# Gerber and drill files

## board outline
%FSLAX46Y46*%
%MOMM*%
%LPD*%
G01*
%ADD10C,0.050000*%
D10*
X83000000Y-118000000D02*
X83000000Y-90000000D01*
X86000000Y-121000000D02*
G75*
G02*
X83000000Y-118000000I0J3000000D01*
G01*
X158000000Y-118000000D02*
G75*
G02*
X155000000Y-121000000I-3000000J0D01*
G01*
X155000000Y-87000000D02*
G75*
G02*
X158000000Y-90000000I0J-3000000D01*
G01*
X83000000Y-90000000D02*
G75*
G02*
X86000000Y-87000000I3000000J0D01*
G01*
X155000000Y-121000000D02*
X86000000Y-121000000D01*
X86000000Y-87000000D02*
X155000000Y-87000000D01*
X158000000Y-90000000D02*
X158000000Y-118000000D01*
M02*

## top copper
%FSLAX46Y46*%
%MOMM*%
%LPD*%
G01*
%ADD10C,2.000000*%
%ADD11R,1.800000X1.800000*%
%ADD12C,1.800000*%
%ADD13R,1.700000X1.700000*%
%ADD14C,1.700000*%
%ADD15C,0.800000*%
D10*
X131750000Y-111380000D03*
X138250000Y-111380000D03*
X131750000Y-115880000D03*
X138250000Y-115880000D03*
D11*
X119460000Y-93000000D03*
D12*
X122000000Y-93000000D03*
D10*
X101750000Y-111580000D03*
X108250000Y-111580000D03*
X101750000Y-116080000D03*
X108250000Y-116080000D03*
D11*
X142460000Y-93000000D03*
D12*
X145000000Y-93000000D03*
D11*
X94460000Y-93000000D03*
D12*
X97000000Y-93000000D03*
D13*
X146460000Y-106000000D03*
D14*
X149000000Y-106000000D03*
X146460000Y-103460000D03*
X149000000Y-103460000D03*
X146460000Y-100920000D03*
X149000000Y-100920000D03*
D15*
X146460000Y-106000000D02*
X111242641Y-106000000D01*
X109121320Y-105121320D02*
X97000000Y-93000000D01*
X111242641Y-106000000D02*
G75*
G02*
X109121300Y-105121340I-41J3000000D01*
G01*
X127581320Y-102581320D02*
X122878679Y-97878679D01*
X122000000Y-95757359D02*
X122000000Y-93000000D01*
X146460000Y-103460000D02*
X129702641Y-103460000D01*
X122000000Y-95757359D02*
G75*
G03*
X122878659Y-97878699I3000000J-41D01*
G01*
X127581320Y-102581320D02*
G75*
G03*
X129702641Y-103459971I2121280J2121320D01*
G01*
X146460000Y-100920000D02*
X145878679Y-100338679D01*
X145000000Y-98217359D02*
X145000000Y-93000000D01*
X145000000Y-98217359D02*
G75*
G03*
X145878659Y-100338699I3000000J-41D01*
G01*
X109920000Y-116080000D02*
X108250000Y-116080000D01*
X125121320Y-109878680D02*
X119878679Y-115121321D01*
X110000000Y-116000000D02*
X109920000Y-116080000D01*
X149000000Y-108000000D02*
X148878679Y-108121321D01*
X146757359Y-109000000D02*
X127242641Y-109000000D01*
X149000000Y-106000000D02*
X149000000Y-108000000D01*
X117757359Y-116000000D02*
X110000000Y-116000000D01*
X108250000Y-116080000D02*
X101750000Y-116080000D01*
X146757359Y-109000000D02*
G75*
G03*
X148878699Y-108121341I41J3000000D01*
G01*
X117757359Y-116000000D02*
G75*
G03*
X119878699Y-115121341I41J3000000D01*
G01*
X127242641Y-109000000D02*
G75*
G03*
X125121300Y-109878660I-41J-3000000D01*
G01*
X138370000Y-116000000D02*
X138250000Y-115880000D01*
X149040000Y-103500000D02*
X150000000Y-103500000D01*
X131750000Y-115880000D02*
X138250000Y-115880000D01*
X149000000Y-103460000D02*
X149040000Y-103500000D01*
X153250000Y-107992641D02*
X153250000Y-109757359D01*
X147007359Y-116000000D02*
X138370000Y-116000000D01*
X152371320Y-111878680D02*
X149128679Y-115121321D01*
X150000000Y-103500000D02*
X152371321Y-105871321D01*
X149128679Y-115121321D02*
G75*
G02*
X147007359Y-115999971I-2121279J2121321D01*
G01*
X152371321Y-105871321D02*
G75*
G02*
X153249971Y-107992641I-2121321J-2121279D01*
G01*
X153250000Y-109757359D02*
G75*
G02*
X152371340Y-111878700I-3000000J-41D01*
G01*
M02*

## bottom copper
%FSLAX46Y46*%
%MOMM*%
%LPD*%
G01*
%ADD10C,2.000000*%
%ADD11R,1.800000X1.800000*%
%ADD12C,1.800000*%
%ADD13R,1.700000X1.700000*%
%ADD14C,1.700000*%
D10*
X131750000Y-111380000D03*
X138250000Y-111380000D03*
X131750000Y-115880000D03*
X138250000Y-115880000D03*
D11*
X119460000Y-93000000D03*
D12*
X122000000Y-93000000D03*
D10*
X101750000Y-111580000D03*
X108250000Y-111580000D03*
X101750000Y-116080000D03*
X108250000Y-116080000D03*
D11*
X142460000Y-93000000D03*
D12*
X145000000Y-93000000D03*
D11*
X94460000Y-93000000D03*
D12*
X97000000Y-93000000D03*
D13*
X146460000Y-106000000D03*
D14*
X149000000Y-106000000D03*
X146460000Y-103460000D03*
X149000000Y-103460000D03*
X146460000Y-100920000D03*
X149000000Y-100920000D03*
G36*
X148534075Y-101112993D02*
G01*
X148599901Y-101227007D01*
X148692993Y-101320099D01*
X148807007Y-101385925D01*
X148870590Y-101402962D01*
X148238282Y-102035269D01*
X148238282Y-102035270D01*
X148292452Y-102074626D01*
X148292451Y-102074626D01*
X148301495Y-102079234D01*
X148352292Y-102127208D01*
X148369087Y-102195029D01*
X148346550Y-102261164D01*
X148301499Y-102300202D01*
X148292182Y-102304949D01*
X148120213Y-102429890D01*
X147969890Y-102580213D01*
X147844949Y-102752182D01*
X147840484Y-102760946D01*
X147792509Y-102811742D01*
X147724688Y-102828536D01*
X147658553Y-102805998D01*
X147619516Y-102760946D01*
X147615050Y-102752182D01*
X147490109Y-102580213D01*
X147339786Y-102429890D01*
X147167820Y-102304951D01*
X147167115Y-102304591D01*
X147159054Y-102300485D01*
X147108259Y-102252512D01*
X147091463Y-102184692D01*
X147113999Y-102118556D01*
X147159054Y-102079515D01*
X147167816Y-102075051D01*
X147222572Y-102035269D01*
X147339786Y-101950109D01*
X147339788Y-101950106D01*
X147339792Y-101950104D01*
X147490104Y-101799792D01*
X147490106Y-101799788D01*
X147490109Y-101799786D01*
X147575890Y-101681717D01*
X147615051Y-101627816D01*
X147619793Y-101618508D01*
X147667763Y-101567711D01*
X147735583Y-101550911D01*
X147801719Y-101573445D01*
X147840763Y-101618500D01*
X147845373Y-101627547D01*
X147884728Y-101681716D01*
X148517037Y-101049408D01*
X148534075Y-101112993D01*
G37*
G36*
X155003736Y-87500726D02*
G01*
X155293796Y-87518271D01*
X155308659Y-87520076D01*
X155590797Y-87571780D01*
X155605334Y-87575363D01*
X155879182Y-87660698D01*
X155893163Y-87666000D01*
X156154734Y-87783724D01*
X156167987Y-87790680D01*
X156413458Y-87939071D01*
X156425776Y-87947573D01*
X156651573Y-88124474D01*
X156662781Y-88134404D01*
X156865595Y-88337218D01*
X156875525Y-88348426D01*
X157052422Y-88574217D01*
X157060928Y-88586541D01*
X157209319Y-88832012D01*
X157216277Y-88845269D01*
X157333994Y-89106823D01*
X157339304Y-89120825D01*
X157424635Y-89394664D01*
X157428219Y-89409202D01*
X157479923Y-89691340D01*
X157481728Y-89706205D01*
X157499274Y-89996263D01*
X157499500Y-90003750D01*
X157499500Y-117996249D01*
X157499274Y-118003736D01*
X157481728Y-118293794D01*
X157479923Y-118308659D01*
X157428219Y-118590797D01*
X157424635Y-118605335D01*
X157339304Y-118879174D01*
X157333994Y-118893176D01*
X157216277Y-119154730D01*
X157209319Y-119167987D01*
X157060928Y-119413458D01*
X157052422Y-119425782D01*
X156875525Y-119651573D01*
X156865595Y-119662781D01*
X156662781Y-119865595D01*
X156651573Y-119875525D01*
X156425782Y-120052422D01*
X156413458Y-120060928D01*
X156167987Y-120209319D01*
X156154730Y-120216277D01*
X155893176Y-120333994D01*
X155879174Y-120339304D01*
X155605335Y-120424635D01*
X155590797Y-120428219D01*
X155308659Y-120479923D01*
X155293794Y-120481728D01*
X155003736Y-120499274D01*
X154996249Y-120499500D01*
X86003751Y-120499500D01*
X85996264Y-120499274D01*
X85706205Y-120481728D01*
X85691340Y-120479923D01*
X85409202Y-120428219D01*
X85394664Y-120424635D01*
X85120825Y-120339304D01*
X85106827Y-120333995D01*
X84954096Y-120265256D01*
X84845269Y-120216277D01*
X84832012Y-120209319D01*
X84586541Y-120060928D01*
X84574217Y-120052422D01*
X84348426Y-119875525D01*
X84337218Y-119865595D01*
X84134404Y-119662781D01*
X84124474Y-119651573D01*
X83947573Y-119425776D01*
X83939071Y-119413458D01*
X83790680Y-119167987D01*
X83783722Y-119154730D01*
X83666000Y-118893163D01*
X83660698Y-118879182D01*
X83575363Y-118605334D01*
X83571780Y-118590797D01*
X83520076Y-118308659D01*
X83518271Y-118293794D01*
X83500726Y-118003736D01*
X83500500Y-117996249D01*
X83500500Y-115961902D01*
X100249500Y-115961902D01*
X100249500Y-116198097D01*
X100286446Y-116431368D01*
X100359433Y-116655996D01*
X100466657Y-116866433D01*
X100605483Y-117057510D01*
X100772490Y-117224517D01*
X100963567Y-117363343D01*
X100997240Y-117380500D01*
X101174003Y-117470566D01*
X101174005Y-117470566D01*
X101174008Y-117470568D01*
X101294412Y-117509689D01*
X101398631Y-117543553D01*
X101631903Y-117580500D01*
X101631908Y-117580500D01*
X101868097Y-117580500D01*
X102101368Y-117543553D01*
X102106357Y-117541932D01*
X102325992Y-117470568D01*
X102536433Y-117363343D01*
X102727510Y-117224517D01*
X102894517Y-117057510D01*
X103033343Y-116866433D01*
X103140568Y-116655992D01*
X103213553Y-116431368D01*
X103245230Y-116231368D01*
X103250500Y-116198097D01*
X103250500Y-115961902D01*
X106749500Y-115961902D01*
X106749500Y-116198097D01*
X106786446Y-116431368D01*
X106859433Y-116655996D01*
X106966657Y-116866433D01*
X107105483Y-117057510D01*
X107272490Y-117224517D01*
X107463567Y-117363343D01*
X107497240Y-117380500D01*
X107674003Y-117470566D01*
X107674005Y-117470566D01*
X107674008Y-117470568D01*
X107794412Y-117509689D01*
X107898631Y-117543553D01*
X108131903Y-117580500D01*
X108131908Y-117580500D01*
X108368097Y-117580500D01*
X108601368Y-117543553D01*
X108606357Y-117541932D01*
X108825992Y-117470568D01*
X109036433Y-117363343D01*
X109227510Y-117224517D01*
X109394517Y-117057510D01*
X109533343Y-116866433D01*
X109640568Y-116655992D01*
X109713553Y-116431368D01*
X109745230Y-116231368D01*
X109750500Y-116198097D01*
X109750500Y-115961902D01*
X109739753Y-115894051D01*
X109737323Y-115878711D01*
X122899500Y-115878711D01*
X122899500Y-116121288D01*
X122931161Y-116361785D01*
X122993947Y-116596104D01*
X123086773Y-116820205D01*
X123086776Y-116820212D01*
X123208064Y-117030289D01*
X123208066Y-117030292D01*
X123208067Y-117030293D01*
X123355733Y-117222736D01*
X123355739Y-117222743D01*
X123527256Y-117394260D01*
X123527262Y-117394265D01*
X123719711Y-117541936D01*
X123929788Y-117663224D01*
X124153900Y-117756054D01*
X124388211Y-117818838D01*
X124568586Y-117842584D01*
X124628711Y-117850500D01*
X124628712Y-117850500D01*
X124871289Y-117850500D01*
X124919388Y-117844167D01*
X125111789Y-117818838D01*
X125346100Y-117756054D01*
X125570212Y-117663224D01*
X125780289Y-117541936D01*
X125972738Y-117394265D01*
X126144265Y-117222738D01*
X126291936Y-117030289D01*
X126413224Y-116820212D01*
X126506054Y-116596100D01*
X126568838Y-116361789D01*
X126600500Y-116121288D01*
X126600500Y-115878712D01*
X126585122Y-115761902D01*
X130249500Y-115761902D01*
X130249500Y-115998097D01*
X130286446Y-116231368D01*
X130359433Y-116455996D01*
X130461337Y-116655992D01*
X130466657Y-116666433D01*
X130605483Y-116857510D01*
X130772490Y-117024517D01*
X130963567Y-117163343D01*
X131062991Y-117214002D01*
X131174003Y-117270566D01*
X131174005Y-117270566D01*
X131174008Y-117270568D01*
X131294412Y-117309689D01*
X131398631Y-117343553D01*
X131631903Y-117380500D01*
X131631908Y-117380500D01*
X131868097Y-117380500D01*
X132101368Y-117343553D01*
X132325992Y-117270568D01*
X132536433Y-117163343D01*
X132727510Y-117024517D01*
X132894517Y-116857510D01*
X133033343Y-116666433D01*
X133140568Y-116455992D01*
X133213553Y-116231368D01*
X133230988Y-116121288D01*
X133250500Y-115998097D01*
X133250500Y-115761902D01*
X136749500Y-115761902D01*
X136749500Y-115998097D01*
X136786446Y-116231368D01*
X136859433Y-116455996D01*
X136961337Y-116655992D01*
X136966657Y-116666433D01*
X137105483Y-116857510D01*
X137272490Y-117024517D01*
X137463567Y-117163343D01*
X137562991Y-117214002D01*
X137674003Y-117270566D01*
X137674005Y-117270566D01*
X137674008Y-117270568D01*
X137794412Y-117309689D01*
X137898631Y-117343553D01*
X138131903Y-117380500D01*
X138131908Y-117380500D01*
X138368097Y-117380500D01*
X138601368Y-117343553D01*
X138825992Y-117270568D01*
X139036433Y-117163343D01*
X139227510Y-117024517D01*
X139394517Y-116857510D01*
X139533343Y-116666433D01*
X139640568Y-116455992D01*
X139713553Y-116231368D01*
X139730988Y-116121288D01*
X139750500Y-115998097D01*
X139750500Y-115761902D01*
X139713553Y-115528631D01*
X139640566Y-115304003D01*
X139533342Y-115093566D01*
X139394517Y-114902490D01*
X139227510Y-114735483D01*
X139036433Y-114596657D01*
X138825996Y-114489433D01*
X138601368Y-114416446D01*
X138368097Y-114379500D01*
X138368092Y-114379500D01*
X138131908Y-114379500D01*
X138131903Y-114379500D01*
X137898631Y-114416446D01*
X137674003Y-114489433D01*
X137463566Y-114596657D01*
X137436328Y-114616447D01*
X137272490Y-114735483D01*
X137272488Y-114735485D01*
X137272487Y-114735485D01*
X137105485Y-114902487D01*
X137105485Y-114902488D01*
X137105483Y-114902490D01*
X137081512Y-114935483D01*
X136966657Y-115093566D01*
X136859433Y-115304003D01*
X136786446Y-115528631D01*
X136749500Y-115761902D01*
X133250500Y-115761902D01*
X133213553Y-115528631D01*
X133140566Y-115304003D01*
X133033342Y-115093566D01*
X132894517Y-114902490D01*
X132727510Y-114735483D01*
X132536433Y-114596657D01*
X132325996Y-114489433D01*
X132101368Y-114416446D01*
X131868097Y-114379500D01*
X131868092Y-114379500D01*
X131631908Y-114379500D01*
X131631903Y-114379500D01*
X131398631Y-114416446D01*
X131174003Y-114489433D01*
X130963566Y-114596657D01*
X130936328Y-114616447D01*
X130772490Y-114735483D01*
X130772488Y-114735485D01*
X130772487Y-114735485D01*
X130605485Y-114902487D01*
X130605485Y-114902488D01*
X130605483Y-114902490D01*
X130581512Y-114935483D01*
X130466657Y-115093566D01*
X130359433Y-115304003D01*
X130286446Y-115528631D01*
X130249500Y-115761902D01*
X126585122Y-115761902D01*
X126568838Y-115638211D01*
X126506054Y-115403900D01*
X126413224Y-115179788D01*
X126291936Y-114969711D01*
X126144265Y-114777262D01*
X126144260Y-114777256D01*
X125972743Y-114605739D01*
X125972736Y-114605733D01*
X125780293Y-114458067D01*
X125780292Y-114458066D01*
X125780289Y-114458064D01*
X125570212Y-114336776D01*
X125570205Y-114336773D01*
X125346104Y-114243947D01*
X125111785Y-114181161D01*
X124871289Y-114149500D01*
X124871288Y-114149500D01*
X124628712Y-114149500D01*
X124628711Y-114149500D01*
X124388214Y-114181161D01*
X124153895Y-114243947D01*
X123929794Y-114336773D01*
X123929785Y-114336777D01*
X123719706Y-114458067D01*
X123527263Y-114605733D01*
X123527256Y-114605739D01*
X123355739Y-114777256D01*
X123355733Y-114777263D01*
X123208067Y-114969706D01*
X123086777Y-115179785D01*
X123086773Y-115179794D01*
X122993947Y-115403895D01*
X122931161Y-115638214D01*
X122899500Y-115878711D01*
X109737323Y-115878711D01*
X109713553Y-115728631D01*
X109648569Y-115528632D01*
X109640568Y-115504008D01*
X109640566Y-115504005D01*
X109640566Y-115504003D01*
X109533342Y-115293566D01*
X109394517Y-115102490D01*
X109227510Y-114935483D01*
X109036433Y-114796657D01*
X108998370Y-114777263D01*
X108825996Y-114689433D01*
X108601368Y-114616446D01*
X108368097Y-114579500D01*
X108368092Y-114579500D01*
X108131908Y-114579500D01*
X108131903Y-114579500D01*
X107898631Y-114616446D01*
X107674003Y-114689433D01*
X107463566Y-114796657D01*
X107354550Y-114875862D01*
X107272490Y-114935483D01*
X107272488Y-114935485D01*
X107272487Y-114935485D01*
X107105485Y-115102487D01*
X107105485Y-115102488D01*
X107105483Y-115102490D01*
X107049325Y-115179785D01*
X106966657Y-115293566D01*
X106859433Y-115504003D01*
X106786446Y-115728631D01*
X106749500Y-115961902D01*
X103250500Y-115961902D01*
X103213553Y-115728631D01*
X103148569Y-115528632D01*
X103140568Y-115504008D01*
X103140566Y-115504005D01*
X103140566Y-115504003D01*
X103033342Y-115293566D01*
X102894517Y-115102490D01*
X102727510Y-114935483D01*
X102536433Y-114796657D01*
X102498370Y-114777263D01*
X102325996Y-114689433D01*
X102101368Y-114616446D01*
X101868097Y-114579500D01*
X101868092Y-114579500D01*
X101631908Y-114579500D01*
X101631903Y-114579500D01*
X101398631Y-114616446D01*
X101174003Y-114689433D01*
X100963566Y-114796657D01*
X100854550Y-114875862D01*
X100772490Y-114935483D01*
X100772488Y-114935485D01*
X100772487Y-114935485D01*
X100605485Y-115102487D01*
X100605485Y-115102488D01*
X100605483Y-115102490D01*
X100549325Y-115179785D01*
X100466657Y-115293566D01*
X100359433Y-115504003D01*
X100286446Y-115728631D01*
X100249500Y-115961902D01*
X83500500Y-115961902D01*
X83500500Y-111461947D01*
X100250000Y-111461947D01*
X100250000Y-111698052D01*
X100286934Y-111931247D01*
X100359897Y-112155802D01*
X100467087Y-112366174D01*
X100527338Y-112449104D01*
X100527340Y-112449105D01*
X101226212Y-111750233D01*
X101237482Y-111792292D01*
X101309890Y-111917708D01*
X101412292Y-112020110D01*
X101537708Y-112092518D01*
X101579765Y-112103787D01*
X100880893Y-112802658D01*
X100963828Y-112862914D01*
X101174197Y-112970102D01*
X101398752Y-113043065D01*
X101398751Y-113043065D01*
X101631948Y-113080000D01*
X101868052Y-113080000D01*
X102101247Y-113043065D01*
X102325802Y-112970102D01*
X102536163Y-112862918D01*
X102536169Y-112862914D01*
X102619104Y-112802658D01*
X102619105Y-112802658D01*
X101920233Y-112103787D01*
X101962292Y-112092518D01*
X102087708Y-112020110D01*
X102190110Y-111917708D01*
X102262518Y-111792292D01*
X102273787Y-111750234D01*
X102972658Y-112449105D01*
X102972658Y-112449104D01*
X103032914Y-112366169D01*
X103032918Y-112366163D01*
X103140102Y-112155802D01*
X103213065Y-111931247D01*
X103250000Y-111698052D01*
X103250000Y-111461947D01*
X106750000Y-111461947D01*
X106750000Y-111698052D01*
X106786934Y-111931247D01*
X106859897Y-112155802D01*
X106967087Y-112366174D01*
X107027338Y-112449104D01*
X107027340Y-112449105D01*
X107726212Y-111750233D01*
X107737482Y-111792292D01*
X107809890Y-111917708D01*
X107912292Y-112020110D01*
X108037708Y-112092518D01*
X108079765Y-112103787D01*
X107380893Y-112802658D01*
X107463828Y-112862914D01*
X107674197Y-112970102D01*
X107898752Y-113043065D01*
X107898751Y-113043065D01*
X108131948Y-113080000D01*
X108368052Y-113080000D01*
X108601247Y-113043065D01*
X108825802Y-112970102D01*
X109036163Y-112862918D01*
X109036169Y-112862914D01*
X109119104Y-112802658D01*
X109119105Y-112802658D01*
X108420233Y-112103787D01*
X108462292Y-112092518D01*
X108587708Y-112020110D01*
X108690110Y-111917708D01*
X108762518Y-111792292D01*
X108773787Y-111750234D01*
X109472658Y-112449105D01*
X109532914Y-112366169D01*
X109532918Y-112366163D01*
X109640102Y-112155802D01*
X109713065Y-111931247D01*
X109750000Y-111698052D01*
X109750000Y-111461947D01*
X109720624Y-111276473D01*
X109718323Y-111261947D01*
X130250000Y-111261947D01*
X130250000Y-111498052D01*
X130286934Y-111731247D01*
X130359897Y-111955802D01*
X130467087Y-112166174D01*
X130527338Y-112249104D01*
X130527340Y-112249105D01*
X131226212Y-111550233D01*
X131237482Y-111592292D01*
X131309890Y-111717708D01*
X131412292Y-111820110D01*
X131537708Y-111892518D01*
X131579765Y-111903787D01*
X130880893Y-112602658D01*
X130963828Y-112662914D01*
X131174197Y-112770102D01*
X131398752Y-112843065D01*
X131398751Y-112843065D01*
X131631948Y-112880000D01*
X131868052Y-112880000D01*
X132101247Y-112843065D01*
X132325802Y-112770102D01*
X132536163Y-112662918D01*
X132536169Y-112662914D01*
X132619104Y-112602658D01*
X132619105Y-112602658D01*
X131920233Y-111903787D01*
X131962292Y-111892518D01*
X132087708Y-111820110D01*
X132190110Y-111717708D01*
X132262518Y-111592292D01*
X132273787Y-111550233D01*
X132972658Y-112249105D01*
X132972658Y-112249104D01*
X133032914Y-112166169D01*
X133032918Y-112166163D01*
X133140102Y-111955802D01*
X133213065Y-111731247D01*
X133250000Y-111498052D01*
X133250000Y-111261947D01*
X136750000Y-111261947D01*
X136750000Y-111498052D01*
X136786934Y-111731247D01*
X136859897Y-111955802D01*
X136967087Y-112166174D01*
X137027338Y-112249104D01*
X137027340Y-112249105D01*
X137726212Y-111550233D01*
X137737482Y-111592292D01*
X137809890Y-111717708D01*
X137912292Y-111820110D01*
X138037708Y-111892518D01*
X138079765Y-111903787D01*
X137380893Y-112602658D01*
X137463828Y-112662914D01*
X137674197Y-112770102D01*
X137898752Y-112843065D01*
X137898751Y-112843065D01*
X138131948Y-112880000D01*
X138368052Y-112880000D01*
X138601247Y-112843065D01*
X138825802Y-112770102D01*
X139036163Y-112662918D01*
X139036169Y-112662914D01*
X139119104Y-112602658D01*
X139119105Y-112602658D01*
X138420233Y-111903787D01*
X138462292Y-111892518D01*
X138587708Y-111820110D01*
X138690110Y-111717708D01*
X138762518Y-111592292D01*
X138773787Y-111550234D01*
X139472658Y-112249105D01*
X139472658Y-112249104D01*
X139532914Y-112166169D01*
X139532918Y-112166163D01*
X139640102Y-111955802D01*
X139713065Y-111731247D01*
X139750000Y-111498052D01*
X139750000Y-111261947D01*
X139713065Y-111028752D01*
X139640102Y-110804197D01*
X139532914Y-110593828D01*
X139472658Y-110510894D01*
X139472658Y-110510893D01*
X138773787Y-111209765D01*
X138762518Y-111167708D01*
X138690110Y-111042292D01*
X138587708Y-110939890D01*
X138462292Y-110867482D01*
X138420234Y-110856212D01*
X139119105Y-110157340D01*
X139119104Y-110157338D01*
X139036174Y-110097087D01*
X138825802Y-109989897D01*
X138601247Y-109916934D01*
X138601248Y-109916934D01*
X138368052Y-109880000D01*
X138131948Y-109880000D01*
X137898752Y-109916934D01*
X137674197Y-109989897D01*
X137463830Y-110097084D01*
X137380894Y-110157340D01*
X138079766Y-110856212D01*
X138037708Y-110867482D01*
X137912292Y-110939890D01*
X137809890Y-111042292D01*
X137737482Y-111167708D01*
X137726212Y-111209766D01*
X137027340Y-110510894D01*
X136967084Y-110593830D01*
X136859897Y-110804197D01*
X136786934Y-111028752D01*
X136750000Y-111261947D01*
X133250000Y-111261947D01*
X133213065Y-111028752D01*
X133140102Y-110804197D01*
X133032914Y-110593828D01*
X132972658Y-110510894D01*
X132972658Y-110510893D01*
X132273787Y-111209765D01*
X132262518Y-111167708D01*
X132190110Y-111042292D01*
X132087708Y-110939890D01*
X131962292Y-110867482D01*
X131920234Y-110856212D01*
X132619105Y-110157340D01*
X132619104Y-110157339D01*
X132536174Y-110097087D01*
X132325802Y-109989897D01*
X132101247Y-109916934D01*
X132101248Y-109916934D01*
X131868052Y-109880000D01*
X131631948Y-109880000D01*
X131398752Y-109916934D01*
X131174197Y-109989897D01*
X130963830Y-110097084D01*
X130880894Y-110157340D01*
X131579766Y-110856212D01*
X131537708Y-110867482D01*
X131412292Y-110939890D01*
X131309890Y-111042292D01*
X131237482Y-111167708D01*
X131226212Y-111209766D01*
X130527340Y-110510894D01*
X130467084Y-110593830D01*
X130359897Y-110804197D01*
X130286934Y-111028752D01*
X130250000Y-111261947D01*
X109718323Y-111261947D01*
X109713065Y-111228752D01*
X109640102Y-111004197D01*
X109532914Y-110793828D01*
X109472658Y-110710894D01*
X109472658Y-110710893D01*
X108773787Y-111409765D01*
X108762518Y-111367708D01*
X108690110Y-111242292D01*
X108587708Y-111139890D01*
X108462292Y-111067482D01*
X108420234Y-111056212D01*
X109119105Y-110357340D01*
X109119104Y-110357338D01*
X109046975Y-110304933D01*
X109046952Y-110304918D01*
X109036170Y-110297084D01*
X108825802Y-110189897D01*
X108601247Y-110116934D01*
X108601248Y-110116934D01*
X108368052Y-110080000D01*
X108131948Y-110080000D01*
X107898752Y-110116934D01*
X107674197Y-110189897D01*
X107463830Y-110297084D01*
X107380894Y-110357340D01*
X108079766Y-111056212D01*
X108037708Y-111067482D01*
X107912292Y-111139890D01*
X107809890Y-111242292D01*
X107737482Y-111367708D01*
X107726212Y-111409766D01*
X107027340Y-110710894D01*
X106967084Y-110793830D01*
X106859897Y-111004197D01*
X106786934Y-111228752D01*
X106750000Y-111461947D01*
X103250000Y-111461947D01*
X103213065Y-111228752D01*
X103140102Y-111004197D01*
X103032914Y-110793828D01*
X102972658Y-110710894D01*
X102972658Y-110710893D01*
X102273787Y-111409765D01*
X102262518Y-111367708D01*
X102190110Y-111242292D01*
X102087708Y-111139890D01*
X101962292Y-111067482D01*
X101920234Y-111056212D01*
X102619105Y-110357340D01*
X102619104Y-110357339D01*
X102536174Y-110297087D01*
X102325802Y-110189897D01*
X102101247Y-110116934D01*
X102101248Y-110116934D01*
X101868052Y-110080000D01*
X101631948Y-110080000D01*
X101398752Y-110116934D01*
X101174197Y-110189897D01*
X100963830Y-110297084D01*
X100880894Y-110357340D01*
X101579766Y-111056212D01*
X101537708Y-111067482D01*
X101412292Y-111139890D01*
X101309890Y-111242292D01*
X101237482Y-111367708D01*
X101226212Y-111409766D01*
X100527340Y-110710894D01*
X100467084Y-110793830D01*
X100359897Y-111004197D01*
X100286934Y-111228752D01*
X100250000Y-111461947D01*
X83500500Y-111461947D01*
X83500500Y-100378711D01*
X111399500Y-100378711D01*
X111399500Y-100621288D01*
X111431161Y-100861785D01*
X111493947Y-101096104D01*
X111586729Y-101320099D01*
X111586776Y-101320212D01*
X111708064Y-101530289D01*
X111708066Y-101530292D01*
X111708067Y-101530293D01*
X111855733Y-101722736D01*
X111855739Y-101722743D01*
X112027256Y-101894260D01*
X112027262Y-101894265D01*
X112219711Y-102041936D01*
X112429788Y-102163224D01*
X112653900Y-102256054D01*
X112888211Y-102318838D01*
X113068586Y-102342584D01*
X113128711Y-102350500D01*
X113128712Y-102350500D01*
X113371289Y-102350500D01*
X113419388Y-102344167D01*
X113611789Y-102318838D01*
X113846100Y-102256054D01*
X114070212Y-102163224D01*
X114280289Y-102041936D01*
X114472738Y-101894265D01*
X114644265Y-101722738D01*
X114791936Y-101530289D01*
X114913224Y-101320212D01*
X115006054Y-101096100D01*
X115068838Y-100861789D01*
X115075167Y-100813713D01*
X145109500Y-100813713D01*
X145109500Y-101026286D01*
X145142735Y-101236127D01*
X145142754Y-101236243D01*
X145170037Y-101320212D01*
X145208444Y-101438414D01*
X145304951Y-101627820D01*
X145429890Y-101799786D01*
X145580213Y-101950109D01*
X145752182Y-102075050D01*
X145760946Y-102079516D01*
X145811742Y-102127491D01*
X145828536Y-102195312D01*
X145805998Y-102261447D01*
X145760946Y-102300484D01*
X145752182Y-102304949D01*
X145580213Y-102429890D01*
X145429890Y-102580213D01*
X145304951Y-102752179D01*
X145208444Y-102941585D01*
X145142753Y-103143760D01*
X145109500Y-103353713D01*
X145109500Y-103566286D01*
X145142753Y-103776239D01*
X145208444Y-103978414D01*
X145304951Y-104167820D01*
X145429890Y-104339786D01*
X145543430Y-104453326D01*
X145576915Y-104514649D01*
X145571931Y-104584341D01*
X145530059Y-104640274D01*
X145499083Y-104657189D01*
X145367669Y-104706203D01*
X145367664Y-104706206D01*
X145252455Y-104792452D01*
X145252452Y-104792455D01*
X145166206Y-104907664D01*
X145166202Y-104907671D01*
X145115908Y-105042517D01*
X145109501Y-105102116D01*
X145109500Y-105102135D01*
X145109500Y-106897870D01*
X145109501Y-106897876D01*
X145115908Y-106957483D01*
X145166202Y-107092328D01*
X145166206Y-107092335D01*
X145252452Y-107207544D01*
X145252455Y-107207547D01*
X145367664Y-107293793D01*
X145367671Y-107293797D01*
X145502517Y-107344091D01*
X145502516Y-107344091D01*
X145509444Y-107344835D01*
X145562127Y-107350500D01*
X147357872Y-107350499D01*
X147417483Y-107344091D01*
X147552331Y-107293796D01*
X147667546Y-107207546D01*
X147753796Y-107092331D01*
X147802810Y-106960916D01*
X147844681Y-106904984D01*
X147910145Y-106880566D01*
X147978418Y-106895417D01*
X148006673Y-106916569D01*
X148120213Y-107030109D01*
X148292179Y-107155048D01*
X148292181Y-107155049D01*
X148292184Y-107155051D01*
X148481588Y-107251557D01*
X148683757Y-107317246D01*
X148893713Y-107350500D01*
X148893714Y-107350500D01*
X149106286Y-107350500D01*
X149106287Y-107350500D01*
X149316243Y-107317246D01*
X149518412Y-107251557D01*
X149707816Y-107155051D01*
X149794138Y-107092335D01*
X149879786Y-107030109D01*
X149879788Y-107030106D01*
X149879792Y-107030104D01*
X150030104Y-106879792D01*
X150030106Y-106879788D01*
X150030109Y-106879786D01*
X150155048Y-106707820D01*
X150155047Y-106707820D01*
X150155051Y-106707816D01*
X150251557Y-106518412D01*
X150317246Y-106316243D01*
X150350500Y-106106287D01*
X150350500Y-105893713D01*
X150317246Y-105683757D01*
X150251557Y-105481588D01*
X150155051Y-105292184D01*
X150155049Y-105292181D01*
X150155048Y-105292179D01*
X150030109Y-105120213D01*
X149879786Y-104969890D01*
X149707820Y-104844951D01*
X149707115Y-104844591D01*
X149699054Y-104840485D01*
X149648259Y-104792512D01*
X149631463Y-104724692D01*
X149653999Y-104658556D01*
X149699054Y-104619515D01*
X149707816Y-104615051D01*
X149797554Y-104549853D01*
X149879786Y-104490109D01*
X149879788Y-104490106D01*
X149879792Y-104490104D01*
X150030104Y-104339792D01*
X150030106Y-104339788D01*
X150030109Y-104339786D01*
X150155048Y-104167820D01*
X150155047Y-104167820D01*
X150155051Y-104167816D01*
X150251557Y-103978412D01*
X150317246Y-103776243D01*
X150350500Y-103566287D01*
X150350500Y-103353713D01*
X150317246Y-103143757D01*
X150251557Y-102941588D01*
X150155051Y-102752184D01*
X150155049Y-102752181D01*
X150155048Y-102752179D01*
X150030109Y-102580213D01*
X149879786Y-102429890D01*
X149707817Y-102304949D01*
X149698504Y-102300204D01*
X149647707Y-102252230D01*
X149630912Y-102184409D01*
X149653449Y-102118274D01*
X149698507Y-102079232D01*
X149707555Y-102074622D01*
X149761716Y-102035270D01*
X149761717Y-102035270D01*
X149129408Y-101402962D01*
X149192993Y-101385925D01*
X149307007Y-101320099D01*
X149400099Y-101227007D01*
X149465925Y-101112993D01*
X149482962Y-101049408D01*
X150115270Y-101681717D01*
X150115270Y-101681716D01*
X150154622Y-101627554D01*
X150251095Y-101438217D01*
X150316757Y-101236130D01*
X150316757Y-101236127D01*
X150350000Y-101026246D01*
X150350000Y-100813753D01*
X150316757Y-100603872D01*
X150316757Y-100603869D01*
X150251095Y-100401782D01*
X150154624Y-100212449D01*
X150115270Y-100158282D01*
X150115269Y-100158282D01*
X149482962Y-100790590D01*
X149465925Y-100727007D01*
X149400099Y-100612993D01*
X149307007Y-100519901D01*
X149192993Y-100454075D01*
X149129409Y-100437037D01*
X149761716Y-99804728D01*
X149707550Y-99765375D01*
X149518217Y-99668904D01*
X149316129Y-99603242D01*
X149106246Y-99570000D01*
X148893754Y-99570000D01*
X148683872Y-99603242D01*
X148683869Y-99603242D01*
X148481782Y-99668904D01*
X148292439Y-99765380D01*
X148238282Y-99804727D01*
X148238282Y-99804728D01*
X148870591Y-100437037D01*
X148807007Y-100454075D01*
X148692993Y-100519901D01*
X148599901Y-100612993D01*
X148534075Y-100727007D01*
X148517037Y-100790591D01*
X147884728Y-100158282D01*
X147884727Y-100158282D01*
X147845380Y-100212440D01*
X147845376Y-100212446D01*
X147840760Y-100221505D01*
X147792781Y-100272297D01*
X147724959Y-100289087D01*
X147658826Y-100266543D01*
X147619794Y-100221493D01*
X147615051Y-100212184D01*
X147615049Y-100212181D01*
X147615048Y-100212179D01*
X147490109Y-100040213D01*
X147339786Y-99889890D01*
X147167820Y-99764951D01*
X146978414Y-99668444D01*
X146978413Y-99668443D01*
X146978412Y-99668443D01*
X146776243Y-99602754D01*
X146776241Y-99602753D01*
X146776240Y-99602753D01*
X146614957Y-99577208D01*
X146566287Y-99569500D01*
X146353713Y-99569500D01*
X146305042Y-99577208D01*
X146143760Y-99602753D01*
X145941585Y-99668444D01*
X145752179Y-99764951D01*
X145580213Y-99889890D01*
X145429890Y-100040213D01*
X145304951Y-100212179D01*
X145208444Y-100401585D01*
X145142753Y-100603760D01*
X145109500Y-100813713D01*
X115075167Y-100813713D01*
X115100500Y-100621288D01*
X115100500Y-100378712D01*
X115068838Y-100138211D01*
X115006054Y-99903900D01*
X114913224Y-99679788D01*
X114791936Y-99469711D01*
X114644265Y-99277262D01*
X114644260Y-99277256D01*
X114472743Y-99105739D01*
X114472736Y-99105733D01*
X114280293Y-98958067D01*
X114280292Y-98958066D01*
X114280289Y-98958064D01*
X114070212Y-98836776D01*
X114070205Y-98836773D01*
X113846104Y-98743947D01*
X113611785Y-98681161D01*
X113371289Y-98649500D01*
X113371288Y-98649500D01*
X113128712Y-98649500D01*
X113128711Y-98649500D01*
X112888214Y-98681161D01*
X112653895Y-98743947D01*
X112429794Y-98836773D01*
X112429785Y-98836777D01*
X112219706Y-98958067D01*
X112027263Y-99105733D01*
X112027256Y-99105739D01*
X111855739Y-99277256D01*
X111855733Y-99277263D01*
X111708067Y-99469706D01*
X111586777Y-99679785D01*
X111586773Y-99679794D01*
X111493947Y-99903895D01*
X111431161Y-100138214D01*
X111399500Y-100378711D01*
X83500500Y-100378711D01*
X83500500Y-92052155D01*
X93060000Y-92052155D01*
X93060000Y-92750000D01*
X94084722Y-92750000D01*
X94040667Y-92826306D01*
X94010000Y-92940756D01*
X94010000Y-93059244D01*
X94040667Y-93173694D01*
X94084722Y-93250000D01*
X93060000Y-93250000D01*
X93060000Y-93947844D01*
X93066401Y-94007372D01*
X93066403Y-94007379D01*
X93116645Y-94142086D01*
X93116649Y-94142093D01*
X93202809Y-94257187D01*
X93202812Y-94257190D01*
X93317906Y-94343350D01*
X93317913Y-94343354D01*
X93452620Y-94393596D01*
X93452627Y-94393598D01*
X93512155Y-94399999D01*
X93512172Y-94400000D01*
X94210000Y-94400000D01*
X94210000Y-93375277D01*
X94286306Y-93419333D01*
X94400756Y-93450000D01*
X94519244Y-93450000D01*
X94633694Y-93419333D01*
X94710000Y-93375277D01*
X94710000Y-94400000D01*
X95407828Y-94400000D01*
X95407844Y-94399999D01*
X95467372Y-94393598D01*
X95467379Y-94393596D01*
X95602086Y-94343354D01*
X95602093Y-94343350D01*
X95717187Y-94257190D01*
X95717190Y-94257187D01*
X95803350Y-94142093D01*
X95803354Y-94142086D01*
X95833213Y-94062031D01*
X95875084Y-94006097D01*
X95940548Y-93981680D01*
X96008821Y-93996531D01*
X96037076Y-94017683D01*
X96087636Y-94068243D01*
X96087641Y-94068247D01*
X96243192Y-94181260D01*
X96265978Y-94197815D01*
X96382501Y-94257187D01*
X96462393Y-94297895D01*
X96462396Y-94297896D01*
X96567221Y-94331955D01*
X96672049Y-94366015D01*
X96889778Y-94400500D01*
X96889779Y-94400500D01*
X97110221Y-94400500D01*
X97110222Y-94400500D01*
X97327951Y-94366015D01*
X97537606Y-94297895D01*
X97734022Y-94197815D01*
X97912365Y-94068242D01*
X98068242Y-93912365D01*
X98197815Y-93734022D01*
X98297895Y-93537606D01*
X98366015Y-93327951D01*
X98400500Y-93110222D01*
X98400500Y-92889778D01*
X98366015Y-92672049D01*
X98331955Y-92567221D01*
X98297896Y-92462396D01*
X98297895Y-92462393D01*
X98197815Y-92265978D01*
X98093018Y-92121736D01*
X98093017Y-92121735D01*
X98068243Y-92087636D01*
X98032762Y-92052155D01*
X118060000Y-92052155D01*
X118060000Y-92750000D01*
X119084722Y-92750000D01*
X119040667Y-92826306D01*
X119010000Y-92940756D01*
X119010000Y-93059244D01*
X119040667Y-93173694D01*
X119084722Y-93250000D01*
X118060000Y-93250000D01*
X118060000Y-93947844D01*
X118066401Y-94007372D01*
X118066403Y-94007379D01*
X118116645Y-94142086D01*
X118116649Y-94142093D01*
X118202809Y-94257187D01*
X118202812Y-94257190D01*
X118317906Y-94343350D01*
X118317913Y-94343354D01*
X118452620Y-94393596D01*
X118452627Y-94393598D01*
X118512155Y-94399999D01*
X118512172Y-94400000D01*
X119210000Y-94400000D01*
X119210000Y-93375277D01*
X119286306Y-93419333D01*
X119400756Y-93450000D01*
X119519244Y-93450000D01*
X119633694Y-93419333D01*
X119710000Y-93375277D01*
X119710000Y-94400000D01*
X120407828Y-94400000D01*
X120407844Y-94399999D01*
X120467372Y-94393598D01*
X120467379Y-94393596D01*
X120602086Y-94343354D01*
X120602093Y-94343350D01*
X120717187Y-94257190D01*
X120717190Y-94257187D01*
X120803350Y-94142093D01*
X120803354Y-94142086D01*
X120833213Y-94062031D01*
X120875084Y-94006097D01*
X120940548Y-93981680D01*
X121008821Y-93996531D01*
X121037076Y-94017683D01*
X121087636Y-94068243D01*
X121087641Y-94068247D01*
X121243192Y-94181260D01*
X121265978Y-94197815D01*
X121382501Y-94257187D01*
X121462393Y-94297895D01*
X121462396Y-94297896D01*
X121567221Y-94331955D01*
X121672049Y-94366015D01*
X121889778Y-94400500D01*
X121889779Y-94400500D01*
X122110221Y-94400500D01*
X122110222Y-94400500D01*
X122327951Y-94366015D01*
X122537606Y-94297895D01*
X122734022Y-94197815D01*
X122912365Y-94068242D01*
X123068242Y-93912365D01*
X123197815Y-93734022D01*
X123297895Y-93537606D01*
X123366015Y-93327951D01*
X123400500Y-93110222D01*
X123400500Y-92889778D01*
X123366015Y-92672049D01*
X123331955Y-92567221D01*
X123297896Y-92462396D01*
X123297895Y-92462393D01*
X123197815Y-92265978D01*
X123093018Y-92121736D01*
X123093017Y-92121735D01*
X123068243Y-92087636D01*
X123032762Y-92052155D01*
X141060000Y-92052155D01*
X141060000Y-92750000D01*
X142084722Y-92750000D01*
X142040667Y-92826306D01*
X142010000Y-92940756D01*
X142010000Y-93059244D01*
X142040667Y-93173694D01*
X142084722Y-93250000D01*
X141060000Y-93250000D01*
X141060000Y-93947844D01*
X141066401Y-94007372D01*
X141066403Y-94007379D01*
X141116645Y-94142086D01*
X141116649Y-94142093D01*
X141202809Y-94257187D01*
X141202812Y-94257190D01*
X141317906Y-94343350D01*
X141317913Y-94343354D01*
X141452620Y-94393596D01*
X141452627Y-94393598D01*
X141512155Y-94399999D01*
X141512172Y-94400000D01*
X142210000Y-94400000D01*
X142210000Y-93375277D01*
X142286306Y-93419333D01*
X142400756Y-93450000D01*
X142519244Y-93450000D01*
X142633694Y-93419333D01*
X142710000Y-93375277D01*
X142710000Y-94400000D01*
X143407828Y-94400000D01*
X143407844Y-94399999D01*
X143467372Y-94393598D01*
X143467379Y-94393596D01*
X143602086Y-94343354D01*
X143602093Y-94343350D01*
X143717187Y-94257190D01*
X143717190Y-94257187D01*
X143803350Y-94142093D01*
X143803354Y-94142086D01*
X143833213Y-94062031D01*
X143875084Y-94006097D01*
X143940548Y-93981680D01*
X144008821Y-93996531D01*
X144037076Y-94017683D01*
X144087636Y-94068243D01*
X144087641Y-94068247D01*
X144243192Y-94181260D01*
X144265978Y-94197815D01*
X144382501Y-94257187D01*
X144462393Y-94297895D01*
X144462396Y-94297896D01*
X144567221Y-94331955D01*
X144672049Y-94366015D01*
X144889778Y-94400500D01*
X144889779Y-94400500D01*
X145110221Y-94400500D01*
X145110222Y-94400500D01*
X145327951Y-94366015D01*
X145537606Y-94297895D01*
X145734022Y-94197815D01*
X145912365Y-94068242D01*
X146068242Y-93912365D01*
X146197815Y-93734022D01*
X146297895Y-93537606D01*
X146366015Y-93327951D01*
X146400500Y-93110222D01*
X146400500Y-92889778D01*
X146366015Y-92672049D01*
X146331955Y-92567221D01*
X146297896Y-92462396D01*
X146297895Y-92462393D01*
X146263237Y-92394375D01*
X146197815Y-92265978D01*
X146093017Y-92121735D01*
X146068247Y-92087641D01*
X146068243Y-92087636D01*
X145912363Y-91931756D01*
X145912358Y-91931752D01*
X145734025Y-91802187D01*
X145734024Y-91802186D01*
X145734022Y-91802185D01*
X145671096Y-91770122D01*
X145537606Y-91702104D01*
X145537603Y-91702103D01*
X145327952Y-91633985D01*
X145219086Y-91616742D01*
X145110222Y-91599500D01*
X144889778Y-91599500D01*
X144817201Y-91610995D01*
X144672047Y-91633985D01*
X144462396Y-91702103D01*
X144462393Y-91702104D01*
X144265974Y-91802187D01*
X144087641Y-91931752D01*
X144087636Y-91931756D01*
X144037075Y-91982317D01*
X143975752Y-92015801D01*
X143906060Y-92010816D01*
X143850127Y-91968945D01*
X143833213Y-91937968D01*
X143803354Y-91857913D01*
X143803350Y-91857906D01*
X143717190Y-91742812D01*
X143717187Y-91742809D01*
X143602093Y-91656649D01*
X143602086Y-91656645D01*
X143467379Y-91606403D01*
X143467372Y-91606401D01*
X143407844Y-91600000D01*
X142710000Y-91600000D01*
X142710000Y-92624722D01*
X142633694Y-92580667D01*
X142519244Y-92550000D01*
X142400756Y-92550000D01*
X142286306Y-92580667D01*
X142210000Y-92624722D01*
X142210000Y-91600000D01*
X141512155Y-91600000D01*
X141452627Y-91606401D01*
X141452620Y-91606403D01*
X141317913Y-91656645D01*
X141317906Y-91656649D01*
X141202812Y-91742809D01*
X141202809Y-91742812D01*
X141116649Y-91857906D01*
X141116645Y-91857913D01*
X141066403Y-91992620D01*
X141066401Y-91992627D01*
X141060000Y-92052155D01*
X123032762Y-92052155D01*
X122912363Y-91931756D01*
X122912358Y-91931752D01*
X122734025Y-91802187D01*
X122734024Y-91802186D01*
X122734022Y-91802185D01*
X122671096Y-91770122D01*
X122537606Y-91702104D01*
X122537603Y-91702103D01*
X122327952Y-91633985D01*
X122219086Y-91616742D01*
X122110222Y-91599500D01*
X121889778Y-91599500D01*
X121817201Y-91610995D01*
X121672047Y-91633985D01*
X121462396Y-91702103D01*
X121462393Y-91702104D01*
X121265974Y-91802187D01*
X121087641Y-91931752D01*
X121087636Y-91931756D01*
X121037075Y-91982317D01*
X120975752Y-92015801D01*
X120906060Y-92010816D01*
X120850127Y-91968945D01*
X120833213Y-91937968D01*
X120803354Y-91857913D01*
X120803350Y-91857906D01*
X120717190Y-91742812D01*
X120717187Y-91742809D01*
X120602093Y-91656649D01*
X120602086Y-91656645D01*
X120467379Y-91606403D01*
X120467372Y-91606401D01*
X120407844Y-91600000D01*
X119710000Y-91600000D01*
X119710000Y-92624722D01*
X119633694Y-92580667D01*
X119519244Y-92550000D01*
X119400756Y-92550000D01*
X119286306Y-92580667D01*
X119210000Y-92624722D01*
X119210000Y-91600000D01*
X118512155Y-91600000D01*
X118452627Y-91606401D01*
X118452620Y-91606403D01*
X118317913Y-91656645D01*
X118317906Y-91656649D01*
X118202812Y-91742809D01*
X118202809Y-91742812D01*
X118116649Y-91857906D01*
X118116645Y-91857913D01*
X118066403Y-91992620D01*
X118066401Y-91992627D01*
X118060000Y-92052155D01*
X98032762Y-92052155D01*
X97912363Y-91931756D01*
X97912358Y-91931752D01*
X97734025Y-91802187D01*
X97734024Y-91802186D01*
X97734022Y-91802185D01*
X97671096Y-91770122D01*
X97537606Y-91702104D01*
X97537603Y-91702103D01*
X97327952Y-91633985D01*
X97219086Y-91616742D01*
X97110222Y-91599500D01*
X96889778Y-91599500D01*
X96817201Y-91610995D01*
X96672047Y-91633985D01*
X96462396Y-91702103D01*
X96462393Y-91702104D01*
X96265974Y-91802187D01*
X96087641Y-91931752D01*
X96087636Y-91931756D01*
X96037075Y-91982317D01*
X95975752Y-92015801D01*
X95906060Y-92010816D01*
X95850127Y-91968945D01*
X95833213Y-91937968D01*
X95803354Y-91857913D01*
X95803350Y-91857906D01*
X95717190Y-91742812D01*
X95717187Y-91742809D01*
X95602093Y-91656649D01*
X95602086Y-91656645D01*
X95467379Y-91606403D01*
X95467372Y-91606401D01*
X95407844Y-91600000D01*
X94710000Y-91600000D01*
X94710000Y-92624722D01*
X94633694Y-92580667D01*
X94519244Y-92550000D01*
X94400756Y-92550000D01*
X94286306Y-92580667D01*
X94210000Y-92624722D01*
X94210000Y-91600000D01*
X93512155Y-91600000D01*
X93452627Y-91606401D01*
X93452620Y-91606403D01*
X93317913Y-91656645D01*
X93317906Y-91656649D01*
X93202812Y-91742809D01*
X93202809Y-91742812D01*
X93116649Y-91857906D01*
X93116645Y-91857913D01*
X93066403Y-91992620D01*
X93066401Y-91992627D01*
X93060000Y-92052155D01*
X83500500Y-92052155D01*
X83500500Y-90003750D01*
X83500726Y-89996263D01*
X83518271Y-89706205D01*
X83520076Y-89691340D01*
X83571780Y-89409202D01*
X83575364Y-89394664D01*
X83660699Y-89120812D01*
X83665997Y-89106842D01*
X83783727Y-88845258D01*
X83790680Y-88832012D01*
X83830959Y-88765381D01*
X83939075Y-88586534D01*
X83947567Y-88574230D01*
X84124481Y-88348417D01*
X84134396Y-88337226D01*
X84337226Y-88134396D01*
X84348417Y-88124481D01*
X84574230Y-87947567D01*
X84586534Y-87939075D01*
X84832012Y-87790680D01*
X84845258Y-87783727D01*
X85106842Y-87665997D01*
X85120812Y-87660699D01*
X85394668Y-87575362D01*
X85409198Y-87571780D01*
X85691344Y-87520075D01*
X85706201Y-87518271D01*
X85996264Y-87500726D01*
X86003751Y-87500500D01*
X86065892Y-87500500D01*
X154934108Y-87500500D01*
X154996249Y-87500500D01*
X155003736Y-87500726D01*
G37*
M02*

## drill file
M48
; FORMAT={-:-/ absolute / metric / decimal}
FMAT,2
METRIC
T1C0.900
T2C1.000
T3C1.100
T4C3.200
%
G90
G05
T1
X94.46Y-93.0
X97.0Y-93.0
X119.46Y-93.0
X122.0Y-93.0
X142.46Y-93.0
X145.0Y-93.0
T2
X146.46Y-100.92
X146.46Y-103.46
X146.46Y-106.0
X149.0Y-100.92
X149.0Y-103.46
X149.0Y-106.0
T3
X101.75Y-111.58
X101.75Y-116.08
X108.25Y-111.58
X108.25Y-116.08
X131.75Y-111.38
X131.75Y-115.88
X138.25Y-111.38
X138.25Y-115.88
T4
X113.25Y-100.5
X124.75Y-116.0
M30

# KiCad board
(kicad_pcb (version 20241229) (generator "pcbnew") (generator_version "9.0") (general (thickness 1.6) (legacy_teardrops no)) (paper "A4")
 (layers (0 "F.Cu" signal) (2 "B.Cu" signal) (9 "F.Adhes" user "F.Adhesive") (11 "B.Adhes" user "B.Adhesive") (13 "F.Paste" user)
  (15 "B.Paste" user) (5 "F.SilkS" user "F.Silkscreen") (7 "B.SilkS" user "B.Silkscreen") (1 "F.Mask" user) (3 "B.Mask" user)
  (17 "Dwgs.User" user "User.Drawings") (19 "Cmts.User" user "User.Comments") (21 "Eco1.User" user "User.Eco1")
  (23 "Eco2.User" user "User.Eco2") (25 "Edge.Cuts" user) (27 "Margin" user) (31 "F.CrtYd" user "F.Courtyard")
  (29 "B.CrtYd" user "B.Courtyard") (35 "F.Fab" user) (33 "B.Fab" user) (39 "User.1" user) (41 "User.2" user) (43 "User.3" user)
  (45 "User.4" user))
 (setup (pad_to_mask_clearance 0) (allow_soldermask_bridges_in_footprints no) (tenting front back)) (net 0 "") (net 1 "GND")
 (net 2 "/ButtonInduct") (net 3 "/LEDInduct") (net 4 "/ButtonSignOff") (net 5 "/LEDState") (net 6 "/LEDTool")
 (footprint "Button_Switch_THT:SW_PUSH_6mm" (layer "F.Cu") (at 131.75 111.38)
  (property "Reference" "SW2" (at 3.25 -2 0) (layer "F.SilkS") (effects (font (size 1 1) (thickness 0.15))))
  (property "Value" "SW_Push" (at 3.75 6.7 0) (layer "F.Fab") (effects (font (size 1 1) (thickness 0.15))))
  (pad "1" thru_hole circle (at 0 0 90) (size 2 2) (drill 1.1) (layers "*.Cu" "*.Mask") (remove_unused_layers no) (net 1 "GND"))
  (pad "1" thru_hole circle (at 6.5 0 90) (size 2 2) (drill 1.1) (layers "*.Cu" "*.Mask") (remove_unused_layers no) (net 1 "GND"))
  (pad "2" thru_hole circle (at 0 4.5 90) (size 2 2) (drill 1.1) (layers "*.Cu" "*.Mask") (remove_unused_layers no) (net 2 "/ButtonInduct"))
  (pad "2" thru_hole circle (at 6.5 4.5 90) (size 2 2) (drill 1.1) (layers "*.Cu" "*.Mask") (remove_unused_layers no)
   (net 2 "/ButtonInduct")))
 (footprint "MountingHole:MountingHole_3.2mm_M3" (layer "F.Cu") (at 124.75 116)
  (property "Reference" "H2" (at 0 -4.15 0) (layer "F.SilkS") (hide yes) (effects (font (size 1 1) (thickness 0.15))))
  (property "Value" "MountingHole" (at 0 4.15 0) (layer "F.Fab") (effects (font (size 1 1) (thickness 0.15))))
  (pad "" np_thru_hole circle (at 0 0) (size 3.2 3.2) (drill 3.2) (layers "*.Cu" "*.Mask")))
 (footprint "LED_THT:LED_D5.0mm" (layer "F.Cu") (at 119.46 93)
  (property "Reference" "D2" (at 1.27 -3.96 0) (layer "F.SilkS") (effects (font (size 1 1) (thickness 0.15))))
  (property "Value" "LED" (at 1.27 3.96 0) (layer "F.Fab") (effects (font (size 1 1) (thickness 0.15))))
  (pad "1" thru_hole rect (at 0 0) (size 1.8 1.8) (drill 0.9) (layers "*.Cu" "*.Mask") (remove_unused_layers no) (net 1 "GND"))
  (pad "2" thru_hole circle (at 2.54 0) (size 1.8 1.8) (drill 0.9) (layers "*.Cu" "*.Mask") (remove_unused_layers no) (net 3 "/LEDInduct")))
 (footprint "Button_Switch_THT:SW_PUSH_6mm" (layer "F.Cu") (at 101.75 111.58)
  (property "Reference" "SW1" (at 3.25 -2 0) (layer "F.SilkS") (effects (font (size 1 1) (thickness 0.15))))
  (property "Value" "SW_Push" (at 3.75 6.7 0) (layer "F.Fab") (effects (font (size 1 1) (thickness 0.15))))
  (pad "1" thru_hole circle (at 0 0 90) (size 2 2) (drill 1.1) (layers "*.Cu" "*.Mask") (remove_unused_layers no) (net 1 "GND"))
  (pad "1" thru_hole circle (at 6.5 0 90) (size 2 2) (drill 1.1) (layers "*.Cu" "*.Mask") (remove_unused_layers no) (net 1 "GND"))
  (pad "2" thru_hole circle (at 0 4.5 90) (size 2 2) (drill 1.1) (layers "*.Cu" "*.Mask") (remove_unused_layers no) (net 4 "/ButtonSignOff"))
  (pad "2" thru_hole circle (at 6.5 4.5 90) (size 2 2) (drill 1.1) (layers "*.Cu" "*.Mask") (remove_unused_layers no)
   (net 4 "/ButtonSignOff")))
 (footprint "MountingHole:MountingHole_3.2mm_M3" (layer "F.Cu") (at 113.25 100.5)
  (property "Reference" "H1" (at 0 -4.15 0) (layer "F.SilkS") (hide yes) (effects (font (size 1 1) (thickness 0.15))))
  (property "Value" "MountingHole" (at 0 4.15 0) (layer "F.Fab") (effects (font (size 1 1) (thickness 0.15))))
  (pad "" np_thru_hole circle (at 0 0) (size 3.2 3.2) (drill 3.2) (layers "*.Cu" "*.Mask")))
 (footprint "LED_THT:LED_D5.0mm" (layer "F.Cu") (at 142.46 93)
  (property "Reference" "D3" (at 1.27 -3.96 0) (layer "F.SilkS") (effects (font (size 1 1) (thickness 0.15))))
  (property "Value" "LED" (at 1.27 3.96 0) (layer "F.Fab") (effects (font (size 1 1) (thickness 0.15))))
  (pad "1" thru_hole rect (at 0 0) (size 1.8 1.8) (drill 0.9) (layers "*.Cu" "*.Mask") (remove_unused_layers no) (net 1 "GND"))
  (pad "2" thru_hole circle (at 2.54 0) (size 1.8 1.8) (drill 0.9) (layers "*.Cu" "*.Mask") (remove_unused_layers no) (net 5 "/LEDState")))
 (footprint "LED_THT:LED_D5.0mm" (layer "F.Cu") (at 94.46 93)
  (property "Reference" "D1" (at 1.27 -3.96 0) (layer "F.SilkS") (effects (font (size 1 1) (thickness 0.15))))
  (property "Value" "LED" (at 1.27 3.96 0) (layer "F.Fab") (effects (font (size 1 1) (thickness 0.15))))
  (pad "1" thru_hole rect (at 0 0) (size 1.8 1.8) (drill 0.9) (layers "*.Cu" "*.Mask") (remove_unused_layers no) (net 1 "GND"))
  (pad "2" thru_hole circle (at 2.54 0) (size 1.8 1.8) (drill 0.9) (layers "*.Cu" "*.Mask") (remove_unused_layers no) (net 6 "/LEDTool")))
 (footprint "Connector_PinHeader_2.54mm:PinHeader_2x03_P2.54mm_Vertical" (layer "B.Cu") (at 146.46 106)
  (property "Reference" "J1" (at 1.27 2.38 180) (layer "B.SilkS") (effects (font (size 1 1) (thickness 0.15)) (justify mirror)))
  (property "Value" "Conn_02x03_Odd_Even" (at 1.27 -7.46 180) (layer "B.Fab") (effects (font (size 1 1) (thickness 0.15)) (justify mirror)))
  (pad "1" thru_hole rect (at 0 0) (size 1.7 1.7) (drill 1) (layers "*.Cu" "*.Mask") (remove_unused_layers no) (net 6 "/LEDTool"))
  (pad "2" thru_hole circle (at 2.54 0) (size 1.7 1.7) (drill 1) (layers "*.Cu" "*.Mask") (remove_unused_layers no) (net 4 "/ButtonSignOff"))
  (pad "3" thru_hole circle (at 0 -2.54) (size 1.7 1.7) (drill 1) (layers "*.Cu" "*.Mask") (remove_unused_layers no) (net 3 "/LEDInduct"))
  (pad "4" thru_hole circle (at 2.54 -2.54) (size 1.7 1.7) (drill 1) (layers "*.Cu" "*.Mask") (remove_unused_layers no)
   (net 2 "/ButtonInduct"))
  (pad "5" thru_hole circle (at 0 -5.08) (size 1.7 1.7) (drill 1) (layers "*.Cu" "*.Mask") (remove_unused_layers no) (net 5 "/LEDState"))
  (pad "6" thru_hole circle (at 2.54 -5.08) (size 1.7 1.7) (drill 1) (layers "*.Cu" "*.Mask") (remove_unused_layers no) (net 1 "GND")))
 (gr_line (start 83 118) (end 83 90) (stroke (width 0.05) (type default)) (layer "Edge.Cuts"))
 (gr_arc (start 86 121) (mid 83.87868 120.12132) (end 83 118) (stroke (width 0.05) (type default)) (layer "Edge.Cuts"))
 (gr_arc (start 158 118) (mid 157.12132 120.12132) (end 155 121) (stroke (width 0.05) (type default)) (layer "Edge.Cuts"))
 (gr_arc (start 155 87) (mid 157.12132 87.87868) (end 158 90) (stroke (width 0.05) (type default)) (layer "Edge.Cuts"))
 (gr_arc (start 83 90) (mid 83.87868 87.87868) (end 86 87) (stroke (width 0.05) (type default)) (layer "Edge.Cuts"))
 (gr_line (start 155 121) (end 86 121) (stroke (width 0.05) (type default)) (layer "Edge.Cuts"))
 (gr_line (start 86 87) (end 155 87) (stroke (width 0.05) (type default)) (layer "Edge.Cuts"))
 (gr_line (start 158 90) (end 158 118) (stroke (width 0.05) (type default)) (layer "Edge.Cuts"))
 (segment (start 146.46 106) (end 111.242641 106) (width 0.8) (layer "F.Cu") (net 6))
 (segment (start 109.12132 105.12132) (end 97 93) (width 0.8) (layer "F.Cu") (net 6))
 (arc (start 111.242641 106) (mid 110.09459 105.771638) (end 109.12132 105.12132) (width 0.8) (layer "F.Cu") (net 6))
 (segment (start 127.58132 102.58132) (end 122.878679 97.878679) (width 0.8) (layer "F.Cu") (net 3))
 (segment (start 122 95.757359) (end 122 93) (width 0.8) (layer "F.Cu") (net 3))
 (segment (start 146.46 103.46) (end 129.702641 103.46) (width 0.8) (layer "F.Cu") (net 3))
 (arc (start 122 95.757359) (mid 122.228361 96.905409) (end 122.878679 97.878679) (width 0.8) (layer "F.Cu") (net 3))
 (arc (start 127.58132 102.58132) (mid 128.55459 103.231639) (end 129.702641 103.46) (width 0.8) (layer "F.Cu") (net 3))
 (segment (start 146.46 100.92) (end 145.878679 100.338679) (width 0.8) (layer "F.Cu") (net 5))
 (segment (start 145 98.217359) (end 145 93) (width 0.8) (layer "F.Cu") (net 5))
 (arc (start 145 98.217359) (mid 145.228361 99.365409) (end 145.878679 100.338679) (width 0.8) (layer "F.Cu") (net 5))
 (segment (start 109.92 116.08) (end 108.25 116.08) (width 0.8) (layer "F.Cu") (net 4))
 (segment (start 125.12132 109.87868) (end 119.878679 115.121321) (width 0.8) (layer "F.Cu") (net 4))
 (segment (start 110 116) (end 109.92 116.08) (width 0.8) (layer "F.Cu") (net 4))
 (segment (start 149 108) (end 148.878679 108.121321) (width 0.8) (layer "F.Cu") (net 4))
 (segment (start 146.757359 109) (end 127.242641 109) (width 0.8) (layer "F.Cu") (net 4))
 (segment (start 149 106) (end 149 108) (width 0.8) (layer "F.Cu") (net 4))
 (segment (start 117.757359 116) (end 110 116) (width 0.8) (layer "F.Cu") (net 4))
 (segment (start 108.25 116.08) (end 101.75 116.08) (width 0.8) (layer "F.Cu") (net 4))
 (arc (start 146.757359 109) (mid 147.905409 108.771639) (end 148.878679 108.121321) (width 0.8) (layer "F.Cu") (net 4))
 (arc (start 117.757359 116) (mid 118.905409 115.771639) (end 119.878679 115.121321) (width 0.8) (layer "F.Cu") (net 4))
 (arc (start 127.242641 109) (mid 126.09459 109.228362) (end 125.12132 109.87868) (width 0.8) (layer "F.Cu") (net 4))
 (segment (start 138.37 116) (end 138.25 115.88) (width 0.8) (layer "F.Cu") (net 2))
 (segment (start 149.04 103.5) (end 150 103.5) (width 0.8) (layer "F.Cu") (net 2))
 (segment (start 131.75 115.88) (end 138.25 115.88) (width 0.8) (layer "F.Cu") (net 2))
 (segment (start 149 103.46) (end 149.04 103.5) (width 0.8) (layer "F.Cu") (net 2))
 (segment (start 153.25 107.992641) (end 153.25 109.757359) (width 0.8) (layer "F.Cu") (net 2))
 (segment (start 147.007359 116) (end 138.37 116) (width 0.8) (layer "F.Cu") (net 2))
 (segment (start 152.37132 111.87868) (end 149.128679 115.121321) (width 0.8) (layer "F.Cu") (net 2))
 (segment (start 150 103.5) (end 152.371321 105.871321) (width 0.8) (layer "F.Cu") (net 2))
 (arc (start 149.128679 115.121321) (mid 148.155409 115.771639) (end 147.007359 116) (width 0.8) (layer "F.Cu") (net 2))
 (arc (start 152.371321 105.871321) (mid 153.021639 106.844591) (end 153.25 107.992641) (width 0.8) (layer "F.Cu") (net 2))
 (arc (start 153.25 109.757359) (mid 153.021639 110.90541) (end 152.37132 111.87868) (width 0.8) (layer "F.Cu") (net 2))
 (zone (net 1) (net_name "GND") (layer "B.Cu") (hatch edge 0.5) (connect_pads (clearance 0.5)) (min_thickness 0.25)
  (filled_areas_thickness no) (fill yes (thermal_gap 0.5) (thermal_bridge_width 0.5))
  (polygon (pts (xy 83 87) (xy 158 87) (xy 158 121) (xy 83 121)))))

